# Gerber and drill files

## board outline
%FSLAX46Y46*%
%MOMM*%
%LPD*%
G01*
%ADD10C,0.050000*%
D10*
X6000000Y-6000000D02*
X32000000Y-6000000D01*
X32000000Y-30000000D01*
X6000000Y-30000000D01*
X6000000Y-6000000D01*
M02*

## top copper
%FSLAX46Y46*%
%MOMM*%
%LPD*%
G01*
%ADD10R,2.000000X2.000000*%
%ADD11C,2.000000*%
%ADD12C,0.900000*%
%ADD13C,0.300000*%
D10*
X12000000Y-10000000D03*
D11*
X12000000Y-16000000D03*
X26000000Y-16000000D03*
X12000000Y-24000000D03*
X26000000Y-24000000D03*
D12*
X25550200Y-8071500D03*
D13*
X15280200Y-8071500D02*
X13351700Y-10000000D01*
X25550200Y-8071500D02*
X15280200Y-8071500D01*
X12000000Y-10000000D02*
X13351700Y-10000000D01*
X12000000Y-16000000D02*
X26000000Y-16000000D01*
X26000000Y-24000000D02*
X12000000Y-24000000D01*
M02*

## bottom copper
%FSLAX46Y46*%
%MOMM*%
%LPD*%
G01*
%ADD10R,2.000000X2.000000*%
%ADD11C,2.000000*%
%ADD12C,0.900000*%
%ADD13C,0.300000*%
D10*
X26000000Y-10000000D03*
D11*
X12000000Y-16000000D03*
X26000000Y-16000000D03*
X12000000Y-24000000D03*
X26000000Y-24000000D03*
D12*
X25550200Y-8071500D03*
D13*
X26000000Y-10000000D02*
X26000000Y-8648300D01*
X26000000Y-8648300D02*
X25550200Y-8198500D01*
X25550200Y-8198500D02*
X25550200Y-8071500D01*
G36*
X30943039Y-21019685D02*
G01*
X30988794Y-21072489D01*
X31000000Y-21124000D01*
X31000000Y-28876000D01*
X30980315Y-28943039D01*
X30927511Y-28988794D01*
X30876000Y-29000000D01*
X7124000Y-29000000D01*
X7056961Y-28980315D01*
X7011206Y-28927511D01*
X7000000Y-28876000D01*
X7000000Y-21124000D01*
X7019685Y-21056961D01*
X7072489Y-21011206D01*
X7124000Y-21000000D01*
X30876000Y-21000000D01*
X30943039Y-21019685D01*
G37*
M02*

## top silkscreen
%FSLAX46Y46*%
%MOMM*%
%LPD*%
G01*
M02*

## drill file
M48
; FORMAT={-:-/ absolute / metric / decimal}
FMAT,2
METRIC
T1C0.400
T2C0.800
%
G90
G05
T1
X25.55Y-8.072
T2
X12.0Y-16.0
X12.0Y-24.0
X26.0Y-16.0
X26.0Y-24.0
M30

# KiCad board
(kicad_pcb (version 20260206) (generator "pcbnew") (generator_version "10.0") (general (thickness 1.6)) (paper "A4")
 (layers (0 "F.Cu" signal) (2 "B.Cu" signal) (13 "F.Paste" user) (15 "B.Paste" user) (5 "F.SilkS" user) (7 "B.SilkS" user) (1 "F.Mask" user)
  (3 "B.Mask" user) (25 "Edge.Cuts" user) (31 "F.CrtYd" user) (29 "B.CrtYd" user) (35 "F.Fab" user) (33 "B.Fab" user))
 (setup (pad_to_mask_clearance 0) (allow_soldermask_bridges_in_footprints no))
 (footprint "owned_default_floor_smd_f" (layer "F.Cu") (at 12 10)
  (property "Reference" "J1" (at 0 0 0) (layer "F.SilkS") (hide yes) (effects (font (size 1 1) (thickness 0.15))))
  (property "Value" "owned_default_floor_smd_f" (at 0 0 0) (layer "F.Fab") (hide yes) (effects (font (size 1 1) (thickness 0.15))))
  (pad "1" smd rect (at 0 0) (size 2 2) (layers "F.Cu" "F.Paste" "F.Mask") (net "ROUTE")))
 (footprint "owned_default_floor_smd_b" (layer "B.Cu") (at 26 10)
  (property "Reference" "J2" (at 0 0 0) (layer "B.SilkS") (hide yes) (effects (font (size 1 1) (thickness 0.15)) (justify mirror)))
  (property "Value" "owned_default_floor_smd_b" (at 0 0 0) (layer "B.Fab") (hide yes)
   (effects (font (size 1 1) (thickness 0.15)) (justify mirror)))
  (pad "1" smd rect (at 0 0) (size 2 2) (layers "B.Cu" "B.Paste" "B.Mask") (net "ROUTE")))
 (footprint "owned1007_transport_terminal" (layer "F.Cu") (at 12 16)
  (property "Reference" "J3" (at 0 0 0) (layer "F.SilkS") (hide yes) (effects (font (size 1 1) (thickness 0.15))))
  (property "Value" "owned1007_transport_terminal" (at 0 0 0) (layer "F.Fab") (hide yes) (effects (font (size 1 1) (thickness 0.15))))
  (pad "1" thru_hole circle (at 0 0) (size 2 2) (drill 0.8) (layers "*.Cu" "*.Mask") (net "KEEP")))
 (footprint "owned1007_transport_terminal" (layer "F.Cu") (at 26 16)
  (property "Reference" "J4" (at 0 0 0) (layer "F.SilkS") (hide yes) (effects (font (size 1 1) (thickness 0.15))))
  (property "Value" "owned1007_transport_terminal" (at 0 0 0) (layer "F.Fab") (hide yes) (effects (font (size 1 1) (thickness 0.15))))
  (pad "1" thru_hole circle (at 0 0) (size 2 2) (drill 0.8) (layers "*.Cu" "*.Mask") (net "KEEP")))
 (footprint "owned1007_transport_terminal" (layer "F.Cu") (at 12 24)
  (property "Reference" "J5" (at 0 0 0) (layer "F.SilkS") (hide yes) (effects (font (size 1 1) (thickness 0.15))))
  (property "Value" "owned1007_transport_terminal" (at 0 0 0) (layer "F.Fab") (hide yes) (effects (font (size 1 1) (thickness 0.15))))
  (pad "1" thru_hole circle (at 0 0) (size 2 2) (drill 0.8) (layers "*.Cu" "*.Mask") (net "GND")))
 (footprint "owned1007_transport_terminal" (layer "F.Cu") (at 26 24)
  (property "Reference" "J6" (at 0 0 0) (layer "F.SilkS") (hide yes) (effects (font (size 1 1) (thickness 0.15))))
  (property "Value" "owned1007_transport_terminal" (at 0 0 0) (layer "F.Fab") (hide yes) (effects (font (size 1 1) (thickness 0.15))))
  (pad "1" thru_hole circle (at 0 0) (size 2 2) (drill 0.8) (layers "*.Cu" "*.Mask") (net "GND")))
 (gr_rect (start 6 6) (end 32 30) (stroke (width 0.05) (type default)) (fill none) (layer "Edge.Cuts"))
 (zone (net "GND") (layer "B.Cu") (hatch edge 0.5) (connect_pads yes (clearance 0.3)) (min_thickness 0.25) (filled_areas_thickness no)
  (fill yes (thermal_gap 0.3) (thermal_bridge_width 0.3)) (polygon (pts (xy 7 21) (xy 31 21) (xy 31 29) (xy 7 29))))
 (segment (start 15.2802 8.0715) (end 13.3517 10) (width 0.3) (layer "F.Cu") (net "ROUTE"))
 (segment (start 25.5502 8.0715) (end 15.2802 8.0715) (width 0.3) (layer "F.Cu") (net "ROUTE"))
 (segment (start 12 10) (end 13.3517 10) (width 0.3) (layer "F.Cu") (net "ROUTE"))
 (via (at 25.5502 8.0715) (size 0.9) (drill 0.4) (layers "F.Cu" "B.Cu") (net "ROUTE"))
 (segment (start 26 10) (end 26 8.6483) (width 0.3) (layer "B.Cu") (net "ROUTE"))
 (segment (start 26 8.6483) (end 25.5502 8.1985) (width 0.3) (layer "B.Cu") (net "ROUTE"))
 (segment (start 25.5502 8.1985) (end 25.5502 8.0715) (width 0.3) (layer "B.Cu") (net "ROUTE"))
 (segment (start 12 16) (end 26 16) (width 0.3) (layer "F.Cu") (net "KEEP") (locked yes))
 (segment (start 26 24) (end 12 24) (width 0.3) (layer "F.Cu") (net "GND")))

